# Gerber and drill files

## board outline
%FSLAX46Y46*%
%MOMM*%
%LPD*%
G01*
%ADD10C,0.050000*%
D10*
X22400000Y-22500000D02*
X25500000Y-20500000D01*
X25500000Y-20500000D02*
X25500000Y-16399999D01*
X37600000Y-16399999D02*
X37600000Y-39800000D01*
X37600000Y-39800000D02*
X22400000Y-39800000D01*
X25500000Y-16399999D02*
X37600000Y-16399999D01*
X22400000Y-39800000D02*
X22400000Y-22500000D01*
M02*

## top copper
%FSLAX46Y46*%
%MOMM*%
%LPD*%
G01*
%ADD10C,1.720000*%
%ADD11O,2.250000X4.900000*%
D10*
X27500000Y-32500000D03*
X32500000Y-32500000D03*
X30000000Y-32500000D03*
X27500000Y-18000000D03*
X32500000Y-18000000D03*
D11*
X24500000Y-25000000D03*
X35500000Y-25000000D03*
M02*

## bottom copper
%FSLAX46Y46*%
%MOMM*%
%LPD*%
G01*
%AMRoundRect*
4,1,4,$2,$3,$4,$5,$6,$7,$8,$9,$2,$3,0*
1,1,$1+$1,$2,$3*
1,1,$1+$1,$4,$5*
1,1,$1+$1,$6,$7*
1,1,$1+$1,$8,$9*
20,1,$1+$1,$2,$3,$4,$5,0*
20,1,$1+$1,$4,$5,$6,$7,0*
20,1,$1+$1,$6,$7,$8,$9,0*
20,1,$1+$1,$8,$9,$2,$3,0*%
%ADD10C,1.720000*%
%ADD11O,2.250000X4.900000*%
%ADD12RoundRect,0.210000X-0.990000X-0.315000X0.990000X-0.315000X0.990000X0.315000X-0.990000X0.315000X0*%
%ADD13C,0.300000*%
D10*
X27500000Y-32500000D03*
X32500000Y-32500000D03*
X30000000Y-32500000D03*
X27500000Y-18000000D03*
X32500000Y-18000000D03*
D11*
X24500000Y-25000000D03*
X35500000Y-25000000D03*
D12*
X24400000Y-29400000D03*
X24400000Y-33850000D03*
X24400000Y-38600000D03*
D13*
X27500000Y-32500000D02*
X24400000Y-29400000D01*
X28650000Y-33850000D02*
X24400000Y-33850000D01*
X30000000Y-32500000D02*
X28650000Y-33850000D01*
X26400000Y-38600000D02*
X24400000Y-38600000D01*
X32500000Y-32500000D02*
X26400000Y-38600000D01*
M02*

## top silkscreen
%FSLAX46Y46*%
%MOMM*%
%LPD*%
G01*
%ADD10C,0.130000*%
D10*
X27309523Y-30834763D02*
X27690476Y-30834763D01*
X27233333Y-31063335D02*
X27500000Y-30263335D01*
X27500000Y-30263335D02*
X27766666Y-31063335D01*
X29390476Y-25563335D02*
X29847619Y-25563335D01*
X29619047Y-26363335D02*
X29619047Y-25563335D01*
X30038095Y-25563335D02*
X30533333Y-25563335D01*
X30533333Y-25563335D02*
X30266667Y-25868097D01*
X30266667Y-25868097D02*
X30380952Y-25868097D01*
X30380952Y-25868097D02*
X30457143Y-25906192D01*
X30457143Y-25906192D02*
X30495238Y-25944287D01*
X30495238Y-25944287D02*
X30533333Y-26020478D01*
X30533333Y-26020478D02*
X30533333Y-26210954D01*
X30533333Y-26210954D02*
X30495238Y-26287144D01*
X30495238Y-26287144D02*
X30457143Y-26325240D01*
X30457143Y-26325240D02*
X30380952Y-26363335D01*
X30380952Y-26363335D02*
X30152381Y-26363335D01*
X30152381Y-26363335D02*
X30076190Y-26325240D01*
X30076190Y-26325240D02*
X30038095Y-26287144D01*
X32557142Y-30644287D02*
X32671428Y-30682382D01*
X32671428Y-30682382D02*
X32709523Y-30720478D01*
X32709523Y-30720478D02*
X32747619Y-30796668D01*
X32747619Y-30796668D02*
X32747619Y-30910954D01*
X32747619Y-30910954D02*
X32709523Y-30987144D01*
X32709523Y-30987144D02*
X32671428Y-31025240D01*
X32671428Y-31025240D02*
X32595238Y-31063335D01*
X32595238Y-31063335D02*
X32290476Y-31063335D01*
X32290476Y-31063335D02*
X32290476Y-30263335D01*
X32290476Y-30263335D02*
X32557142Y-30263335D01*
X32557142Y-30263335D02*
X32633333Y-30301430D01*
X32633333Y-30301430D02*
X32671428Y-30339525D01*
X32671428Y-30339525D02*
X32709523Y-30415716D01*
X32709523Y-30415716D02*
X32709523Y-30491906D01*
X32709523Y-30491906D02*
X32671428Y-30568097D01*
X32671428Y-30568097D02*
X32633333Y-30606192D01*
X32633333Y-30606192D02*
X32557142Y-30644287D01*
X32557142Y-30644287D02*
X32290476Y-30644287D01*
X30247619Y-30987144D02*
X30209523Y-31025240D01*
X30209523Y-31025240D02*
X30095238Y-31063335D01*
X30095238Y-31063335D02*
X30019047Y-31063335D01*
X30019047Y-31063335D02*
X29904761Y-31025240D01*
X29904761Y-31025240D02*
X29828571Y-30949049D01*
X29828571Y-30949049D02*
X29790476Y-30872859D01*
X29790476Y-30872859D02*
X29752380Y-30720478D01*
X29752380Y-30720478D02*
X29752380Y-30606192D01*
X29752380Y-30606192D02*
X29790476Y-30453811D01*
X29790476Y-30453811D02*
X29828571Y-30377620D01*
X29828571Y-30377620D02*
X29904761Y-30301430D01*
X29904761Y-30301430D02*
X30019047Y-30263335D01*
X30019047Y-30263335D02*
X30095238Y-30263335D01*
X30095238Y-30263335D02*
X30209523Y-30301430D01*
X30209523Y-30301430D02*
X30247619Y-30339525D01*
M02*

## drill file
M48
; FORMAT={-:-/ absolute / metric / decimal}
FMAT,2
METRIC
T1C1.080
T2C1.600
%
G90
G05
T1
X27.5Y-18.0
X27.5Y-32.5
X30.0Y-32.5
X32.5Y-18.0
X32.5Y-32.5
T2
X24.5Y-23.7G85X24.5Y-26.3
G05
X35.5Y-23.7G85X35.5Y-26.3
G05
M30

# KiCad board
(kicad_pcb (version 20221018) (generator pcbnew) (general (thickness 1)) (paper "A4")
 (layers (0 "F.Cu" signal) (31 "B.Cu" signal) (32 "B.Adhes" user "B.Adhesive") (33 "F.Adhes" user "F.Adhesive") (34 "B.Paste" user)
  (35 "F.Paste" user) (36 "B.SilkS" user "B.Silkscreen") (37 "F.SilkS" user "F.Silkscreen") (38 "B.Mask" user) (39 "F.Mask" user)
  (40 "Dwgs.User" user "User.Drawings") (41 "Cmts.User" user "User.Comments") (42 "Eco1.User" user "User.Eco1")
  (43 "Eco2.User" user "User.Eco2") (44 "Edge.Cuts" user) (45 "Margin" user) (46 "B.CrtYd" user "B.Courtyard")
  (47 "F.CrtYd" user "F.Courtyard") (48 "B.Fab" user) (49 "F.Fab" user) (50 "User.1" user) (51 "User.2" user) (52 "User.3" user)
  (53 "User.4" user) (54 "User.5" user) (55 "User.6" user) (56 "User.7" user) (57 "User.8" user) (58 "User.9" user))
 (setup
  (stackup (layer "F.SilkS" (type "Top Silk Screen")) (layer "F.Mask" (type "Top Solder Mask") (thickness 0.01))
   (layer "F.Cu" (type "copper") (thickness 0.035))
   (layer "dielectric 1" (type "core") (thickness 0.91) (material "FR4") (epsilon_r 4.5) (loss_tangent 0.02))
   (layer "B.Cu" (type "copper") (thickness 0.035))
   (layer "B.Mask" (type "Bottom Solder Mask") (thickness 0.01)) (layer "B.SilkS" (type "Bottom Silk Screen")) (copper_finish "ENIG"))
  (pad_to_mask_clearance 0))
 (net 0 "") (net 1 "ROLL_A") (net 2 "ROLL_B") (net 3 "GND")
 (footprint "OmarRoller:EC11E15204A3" (layer "F.Cu") (at 30 25)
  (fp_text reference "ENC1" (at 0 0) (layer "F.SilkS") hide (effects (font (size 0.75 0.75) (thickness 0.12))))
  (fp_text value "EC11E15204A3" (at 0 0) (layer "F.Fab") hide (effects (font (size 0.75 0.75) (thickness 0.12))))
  (pad "A" thru_hole circle (at -2.5 7.5) (size 1.72 1.72) (drill 1.08) (layers "*.Cu" "*.Mask") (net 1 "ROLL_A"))
  (pad "B" thru_hole circle (at 2.5 7.5) (size 1.72 1.72) (drill 1.08) (layers "*.Cu" "*.Mask") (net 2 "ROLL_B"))
  (pad "C" thru_hole circle (at 0 7.5) (size 1.72 1.72) (drill 1.08) (layers "*.Cu" "*.Mask") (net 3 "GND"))
  (pad "D" thru_hole circle (at -2.5 -7) (size 1.72 1.72) (drill 1.08) (layers "*.Cu" "*.Mask"))
  (pad "E" thru_hole circle (at 2.5 -7) (size 1.72 1.72) (drill 1.08) (layers "*.Cu" "*.Mask"))
  (pad "M1" thru_hole oval (at -5.5 0) (size 2.25 4.9) (drill oval 1.6 4.2) (layers "*.Cu" "*.Mask"))
  (pad "M2" thru_hole oval (at 5.5 0) (size 2.25 4.9) (drill oval 1.6 4.2) (layers "*.Cu" "*.Mask")))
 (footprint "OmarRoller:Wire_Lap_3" (layer "F.Cu") (at 30 25)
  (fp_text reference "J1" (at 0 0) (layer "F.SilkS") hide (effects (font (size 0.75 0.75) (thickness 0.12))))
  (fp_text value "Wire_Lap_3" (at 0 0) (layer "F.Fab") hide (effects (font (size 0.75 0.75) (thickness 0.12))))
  (pad "1" smd roundrect (at -5.6 4.4) (size 2.4 1.05) (layers "B.Cu" "B.Mask") (roundrect_rratio 0.2) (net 1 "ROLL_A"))
  (pad "2" smd roundrect (at -5.6 8.85) (size 2.4 1.05) (layers "B.Cu" "B.Mask") (roundrect_rratio 0.2) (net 3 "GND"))
  (pad "3" smd roundrect (at -5.6 13.6) (size 2.4 1.05) (layers "B.Cu" "B.Mask") (roundrect_rratio 0.2) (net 2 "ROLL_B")))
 (gr_line (start 22.4 22.5) (end 25.5 20.5) (stroke (width 0.05) (type default)) (layer "Edge.Cuts"))
 (gr_line (start 25.5 20.5) (end 25.5 16.399999) (stroke (width 0.05) (type default)) (layer "Edge.Cuts"))
 (gr_line (start 37.6 16.399999) (end 37.6 39.8) (stroke (width 0.05) (type default)) (layer "Edge.Cuts"))
 (gr_line (start 37.6 39.8) (end 22.4 39.8) (stroke (width 0.05) (type default)) (layer "Edge.Cuts"))
 (gr_line (start 25.5 16.399999) (end 37.6 16.399999) (stroke (width 0.05) (type default)) (layer "Edge.Cuts"))
 (gr_line (start 22.4 39.8) (end 22.4 22.5) (stroke (width 0.05) (type default)) (layer "Edge.Cuts"))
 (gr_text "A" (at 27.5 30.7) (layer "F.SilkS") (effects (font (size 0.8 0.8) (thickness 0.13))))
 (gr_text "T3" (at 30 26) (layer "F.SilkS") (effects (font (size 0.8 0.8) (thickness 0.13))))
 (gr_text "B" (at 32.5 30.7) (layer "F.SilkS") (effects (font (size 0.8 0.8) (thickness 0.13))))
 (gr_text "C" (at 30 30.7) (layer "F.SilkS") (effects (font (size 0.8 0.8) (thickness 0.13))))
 (segment (start 27.5 32.5) (end 24.4 29.4) (width 0.3) (layer "B.Cu") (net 1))
 (segment (start 28.65 33.85) (end 24.4 33.85) (width 0.3) (layer "B.Cu") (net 3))
 (segment (start 30 32.5) (end 28.65 33.85) (width 0.3) (layer "B.Cu") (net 3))
 (segment (start 26.4 38.6) (end 24.4 38.6) (width 0.3) (layer "B.Cu") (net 2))
 (segment (start 32.5 32.5) (end 26.4 38.6) (width 0.3) (layer "B.Cu") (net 2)))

